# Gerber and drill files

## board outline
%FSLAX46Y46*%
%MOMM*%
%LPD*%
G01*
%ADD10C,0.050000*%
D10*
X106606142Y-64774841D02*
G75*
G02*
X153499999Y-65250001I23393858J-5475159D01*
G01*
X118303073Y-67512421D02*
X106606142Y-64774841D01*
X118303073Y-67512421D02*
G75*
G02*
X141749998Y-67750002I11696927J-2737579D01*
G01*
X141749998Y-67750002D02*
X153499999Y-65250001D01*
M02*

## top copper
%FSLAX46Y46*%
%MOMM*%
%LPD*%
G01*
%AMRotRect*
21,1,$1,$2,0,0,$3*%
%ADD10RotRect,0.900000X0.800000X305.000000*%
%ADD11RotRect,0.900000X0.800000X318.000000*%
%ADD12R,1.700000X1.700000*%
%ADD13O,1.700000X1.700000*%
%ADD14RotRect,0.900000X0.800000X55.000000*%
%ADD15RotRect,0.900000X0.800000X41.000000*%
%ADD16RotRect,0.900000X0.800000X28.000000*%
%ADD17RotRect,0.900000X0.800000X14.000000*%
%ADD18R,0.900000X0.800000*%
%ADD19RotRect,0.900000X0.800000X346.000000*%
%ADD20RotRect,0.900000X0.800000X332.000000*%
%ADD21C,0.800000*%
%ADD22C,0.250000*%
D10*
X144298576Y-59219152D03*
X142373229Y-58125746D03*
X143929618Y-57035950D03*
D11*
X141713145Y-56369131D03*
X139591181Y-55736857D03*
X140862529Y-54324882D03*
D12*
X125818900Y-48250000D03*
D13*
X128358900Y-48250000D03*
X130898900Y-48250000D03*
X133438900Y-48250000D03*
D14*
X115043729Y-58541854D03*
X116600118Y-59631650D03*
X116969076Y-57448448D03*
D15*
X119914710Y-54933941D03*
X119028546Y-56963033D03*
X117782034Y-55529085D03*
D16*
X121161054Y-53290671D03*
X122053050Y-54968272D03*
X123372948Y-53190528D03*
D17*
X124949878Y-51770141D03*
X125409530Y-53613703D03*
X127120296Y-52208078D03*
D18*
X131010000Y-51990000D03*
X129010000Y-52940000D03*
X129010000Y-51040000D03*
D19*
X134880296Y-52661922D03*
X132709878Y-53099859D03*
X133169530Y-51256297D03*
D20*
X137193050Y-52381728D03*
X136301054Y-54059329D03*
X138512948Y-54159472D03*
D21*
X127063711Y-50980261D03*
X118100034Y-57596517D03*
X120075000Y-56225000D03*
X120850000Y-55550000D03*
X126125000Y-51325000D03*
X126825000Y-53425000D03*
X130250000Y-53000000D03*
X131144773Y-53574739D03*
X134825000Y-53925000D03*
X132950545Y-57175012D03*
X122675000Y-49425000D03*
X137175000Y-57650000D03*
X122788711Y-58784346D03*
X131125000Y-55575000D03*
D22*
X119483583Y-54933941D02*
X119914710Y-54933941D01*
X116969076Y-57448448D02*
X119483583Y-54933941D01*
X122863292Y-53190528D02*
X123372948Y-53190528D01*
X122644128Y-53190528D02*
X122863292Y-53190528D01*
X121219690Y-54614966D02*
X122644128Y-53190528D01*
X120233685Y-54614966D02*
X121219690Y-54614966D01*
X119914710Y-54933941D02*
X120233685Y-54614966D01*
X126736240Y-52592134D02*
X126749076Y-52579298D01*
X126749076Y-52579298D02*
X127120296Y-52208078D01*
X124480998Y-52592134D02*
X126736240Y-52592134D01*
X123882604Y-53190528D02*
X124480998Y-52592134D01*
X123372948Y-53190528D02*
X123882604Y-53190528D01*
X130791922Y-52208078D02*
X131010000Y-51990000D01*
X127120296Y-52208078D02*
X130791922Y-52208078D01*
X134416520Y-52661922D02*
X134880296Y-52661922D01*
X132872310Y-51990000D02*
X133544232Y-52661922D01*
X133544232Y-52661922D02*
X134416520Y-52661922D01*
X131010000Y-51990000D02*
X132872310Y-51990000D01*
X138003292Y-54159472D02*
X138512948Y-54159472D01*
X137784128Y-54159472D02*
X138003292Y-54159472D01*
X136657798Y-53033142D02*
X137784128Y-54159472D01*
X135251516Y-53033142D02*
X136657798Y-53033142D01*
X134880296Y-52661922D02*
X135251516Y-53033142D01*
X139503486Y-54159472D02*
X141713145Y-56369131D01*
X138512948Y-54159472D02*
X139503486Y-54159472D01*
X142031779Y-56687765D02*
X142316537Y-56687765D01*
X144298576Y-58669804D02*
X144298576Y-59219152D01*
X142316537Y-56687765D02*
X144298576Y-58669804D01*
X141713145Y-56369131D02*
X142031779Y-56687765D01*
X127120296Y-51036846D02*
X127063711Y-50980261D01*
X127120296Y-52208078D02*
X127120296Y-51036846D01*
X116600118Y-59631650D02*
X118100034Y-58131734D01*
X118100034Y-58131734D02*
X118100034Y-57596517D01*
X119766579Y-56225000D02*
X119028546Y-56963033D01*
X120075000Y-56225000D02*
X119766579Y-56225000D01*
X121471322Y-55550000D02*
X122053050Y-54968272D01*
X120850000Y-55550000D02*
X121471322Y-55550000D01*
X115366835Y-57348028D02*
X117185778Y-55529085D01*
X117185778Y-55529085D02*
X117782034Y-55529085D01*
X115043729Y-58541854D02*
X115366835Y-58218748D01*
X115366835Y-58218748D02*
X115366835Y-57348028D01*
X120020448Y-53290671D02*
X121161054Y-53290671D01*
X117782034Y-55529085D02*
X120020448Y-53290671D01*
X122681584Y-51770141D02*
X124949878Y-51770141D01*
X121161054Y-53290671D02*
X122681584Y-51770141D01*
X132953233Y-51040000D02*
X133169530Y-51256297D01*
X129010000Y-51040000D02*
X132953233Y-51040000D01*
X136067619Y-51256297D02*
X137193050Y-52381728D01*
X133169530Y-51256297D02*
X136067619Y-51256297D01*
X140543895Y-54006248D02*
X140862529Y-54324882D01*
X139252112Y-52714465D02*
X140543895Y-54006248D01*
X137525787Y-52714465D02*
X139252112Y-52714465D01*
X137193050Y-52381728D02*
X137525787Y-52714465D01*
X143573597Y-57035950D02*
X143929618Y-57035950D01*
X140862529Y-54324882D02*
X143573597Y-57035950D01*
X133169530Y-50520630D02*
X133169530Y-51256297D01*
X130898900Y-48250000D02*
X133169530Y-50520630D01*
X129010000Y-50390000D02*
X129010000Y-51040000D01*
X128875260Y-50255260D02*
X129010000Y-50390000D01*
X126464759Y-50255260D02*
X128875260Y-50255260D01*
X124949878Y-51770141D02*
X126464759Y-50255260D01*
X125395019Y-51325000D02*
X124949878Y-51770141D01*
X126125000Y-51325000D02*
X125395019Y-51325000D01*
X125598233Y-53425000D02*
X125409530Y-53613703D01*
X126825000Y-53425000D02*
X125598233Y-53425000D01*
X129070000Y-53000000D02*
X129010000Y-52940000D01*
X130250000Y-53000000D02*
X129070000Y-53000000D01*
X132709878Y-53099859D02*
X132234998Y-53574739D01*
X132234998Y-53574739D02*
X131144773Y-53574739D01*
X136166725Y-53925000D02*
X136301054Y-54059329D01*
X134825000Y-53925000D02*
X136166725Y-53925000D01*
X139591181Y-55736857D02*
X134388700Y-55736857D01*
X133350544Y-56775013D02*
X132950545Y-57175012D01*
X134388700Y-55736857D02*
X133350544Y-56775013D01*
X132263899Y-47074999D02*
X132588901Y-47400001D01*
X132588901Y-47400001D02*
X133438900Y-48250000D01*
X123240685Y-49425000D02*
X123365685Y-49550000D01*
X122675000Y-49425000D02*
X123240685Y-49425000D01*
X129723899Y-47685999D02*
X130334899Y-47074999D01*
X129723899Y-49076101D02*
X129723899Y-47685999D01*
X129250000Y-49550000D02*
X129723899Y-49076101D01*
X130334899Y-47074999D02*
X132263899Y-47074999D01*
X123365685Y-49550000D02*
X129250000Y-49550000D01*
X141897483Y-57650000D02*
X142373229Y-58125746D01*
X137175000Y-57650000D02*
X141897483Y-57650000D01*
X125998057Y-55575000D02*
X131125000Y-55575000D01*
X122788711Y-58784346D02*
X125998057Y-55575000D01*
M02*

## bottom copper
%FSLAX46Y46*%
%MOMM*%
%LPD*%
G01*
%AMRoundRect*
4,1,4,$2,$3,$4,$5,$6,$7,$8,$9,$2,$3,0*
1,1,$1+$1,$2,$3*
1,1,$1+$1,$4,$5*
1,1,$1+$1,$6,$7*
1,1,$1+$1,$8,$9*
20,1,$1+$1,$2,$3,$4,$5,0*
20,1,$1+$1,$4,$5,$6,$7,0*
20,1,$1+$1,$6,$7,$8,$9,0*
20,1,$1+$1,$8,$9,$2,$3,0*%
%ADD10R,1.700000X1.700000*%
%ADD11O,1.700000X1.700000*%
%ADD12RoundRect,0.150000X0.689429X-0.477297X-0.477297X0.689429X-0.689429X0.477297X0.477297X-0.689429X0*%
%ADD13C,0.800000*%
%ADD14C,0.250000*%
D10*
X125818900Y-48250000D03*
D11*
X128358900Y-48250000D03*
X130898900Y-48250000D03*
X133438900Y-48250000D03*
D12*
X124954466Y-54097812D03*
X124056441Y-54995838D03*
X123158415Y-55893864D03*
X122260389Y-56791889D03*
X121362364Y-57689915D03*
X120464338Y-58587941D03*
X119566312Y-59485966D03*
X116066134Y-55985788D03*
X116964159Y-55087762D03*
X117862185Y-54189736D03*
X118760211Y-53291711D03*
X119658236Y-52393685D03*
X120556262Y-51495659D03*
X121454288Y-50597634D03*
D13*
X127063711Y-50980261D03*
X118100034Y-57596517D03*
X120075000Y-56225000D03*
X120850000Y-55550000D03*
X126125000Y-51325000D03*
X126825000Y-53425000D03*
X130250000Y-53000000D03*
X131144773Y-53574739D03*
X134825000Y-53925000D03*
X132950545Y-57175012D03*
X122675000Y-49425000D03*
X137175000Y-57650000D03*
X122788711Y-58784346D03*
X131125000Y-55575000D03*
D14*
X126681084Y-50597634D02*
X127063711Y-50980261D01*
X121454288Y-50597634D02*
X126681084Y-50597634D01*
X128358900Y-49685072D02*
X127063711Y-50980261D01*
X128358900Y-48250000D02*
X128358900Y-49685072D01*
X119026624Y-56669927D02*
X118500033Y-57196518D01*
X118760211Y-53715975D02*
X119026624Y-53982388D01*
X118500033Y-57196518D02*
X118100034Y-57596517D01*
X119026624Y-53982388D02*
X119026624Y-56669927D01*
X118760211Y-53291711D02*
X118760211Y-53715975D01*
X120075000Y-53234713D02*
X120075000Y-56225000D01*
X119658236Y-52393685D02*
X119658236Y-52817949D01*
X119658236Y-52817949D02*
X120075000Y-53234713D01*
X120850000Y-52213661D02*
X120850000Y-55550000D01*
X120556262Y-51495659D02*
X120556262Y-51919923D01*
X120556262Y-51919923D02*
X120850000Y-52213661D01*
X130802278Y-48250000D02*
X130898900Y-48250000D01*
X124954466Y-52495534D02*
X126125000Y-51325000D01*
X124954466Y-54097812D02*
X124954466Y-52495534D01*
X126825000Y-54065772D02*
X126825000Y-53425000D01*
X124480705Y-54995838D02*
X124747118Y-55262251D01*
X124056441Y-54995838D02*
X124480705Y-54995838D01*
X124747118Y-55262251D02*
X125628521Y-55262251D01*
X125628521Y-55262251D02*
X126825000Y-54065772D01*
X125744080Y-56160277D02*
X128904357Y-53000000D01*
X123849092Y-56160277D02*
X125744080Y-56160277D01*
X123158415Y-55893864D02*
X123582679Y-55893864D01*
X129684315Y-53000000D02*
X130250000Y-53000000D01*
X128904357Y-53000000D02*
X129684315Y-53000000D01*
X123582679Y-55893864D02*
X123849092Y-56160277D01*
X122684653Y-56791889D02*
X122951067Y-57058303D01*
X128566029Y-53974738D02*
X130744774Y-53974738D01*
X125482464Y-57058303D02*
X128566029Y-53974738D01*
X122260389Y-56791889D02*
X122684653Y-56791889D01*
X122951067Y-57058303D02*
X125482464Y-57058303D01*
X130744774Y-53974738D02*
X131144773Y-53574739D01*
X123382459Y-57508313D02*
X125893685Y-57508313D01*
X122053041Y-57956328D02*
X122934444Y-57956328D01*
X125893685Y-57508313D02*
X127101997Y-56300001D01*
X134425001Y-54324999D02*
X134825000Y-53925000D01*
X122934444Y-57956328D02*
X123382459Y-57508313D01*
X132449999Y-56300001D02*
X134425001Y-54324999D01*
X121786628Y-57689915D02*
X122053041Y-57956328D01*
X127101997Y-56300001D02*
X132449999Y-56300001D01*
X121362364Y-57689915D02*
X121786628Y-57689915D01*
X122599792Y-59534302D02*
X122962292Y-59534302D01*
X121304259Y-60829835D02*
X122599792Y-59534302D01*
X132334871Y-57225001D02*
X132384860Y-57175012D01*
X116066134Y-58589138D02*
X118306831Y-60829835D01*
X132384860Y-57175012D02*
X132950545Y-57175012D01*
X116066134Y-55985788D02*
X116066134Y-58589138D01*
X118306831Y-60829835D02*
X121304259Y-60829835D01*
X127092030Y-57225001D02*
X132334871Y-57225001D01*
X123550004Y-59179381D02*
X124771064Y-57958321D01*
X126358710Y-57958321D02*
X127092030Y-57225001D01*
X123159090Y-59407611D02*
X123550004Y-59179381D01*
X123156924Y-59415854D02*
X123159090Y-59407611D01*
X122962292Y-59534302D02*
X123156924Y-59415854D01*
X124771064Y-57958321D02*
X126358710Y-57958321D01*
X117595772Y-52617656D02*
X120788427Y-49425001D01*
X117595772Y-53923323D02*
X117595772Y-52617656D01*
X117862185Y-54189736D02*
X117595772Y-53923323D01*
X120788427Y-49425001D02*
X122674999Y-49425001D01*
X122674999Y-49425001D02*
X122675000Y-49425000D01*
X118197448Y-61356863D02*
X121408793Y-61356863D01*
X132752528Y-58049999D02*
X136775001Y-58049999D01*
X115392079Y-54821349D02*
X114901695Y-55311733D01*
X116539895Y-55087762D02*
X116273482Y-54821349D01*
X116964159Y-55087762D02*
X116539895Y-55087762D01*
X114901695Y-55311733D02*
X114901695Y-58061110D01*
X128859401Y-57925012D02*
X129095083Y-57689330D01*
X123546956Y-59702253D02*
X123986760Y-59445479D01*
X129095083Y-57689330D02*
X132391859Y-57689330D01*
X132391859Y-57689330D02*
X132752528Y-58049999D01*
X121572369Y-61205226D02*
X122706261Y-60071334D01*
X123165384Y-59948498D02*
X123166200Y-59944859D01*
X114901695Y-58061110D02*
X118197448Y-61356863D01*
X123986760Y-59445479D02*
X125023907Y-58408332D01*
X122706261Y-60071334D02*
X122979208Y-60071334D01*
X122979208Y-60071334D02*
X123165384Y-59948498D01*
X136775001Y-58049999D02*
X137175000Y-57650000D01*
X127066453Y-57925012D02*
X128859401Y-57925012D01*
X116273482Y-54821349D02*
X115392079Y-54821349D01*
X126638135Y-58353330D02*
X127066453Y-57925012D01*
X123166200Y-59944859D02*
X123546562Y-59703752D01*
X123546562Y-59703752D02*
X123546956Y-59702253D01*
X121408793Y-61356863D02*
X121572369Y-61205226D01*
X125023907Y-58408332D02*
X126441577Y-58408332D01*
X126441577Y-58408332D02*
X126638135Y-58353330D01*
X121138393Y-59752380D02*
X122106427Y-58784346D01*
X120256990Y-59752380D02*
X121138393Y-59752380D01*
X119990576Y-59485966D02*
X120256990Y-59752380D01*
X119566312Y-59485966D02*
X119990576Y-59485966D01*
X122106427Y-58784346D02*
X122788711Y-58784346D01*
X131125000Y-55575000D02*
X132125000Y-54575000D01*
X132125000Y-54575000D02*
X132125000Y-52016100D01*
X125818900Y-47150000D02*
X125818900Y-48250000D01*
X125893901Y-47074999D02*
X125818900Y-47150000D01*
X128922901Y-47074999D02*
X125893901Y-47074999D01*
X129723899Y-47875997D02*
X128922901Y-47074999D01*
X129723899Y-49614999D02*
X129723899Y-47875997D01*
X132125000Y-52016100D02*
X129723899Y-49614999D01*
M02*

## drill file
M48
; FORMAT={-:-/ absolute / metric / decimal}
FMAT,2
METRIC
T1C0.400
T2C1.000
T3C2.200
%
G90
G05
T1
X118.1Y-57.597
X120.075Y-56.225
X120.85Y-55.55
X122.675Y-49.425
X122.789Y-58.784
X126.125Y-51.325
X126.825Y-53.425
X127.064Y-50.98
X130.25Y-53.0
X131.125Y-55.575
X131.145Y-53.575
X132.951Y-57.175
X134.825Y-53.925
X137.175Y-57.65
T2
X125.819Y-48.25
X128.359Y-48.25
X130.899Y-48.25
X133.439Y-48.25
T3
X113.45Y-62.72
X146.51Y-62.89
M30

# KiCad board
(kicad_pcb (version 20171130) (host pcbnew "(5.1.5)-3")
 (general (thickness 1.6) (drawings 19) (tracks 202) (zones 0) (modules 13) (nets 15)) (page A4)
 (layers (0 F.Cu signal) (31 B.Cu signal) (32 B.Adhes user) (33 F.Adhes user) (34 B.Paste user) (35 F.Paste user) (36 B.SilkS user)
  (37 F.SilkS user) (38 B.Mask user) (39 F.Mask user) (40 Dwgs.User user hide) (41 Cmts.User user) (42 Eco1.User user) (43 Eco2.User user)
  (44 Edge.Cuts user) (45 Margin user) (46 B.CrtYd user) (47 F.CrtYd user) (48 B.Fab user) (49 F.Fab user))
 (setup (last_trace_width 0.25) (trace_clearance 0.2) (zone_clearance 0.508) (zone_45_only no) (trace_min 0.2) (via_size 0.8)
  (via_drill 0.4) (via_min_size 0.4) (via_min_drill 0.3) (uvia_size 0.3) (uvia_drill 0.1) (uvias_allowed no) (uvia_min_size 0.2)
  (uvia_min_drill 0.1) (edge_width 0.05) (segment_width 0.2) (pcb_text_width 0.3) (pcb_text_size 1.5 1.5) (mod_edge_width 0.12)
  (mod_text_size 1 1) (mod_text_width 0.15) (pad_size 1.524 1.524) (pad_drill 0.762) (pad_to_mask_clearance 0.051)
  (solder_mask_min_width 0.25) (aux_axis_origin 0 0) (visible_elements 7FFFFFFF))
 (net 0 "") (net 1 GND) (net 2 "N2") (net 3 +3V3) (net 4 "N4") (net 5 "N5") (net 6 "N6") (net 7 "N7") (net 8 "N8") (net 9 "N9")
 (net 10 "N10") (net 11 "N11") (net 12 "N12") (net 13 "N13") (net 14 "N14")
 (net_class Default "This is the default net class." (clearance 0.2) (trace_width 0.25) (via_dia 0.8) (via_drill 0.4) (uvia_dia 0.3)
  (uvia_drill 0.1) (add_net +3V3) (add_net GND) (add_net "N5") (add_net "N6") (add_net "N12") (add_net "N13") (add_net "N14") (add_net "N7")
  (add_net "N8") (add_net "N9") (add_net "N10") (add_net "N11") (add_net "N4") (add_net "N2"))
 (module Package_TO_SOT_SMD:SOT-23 (layer F.Cu) (at 143.725 58.4 305)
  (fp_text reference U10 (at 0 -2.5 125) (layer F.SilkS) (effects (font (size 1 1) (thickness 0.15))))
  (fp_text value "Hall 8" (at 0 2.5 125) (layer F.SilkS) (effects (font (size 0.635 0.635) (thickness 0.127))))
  (pad 3 smd rect (at 1 0 305) (size 0.9 0.8) (layers F.Cu F.Paste F.Mask) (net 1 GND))
  (pad 2 smd rect (at -1 0.95 305) (size 0.9 0.8) (layers F.Cu F.Paste F.Mask) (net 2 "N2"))
  (pad 1 smd rect (at -1 -0.95 305) (size 0.9 0.8) (layers F.Cu F.Paste F.Mask) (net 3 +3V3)))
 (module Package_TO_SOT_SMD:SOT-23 (layer F.Cu) (at 140.97 55.7 318)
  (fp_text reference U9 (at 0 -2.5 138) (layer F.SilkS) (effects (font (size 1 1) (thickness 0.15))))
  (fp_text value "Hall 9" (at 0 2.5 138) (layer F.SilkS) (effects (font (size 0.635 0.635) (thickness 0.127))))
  (pad 3 smd rect (at 1 0 318) (size 0.9 0.8) (layers F.Cu F.Paste F.Mask) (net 1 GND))
  (pad 2 smd rect (at -1 0.95 318) (size 0.9 0.8) (layers F.Cu F.Paste F.Mask) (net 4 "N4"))
  (pad 1 smd rect (at -1 -0.95 318) (size 0.9 0.8) (layers F.Cu F.Paste F.Mask) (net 3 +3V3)))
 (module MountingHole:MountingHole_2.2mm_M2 (layer F.Cu) (at 146.51 62.89)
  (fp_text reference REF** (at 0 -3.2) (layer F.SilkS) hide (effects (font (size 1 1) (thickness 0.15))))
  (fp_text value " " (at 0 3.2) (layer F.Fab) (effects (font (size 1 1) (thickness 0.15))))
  (pad 1 np_thru_hole circle (at 0 0) (size 2.2 2.2) (drill 2.2) (layers *.Cu *.Mask)))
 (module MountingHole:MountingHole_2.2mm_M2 (layer F.Cu) (at 113.45 62.72)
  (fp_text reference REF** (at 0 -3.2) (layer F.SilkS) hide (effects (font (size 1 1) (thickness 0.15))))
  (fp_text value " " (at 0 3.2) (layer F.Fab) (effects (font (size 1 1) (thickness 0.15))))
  (pad 1 np_thru_hole circle (at 0 0) (size 2.2 2.2) (drill 2.2) (layers *.Cu *.Mask)))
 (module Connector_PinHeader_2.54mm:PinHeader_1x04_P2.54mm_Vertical (layer F.Cu) (at 125.8189 48.25 90)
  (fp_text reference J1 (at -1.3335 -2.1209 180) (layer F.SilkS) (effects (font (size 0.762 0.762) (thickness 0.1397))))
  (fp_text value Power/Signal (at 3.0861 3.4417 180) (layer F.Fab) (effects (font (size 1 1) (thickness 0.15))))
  (pad 1 thru_hole rect (at 0 0 90) (size 1.7 1.7) (drill 1) (layers *.Cu *.Mask) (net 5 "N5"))
  (pad 2 thru_hole oval (at 0 2.54 90) (size 1.7 1.7) (drill 1) (layers *.Cu *.Mask) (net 1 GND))
  (pad 3 thru_hole oval (at 0 5.08 90) (size 1.7 1.7) (drill 1) (layers *.Cu *.Mask) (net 3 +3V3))
  (pad 4 thru_hole oval (at 0 7.62 90) (size 1.7 1.7) (drill 1) (layers *.Cu *.Mask) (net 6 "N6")))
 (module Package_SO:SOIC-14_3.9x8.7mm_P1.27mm (layer B.Cu) (at 120.5103 55.0418 135)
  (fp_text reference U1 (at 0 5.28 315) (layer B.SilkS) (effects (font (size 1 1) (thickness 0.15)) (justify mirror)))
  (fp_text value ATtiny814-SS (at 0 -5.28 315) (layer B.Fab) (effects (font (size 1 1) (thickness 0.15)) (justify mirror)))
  (pad 1 smd roundrect (at -2.475 3.81 135) (size 1.95 0.6) (layers B.Cu B.Paste B.Mask) (roundrect_rratio 0.25) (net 3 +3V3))
  (pad 2 smd roundrect (at -2.475 2.54 135) (size 1.95 0.6) (layers B.Cu B.Paste B.Mask) (roundrect_rratio 0.25) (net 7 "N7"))
  (pad 3 smd roundrect (at -2.475 1.27 135) (size 1.95 0.6) (layers B.Cu B.Paste B.Mask) (roundrect_rratio 0.25) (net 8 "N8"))
  (pad 4 smd roundrect (at -2.475 0 135) (size 1.95 0.6) (layers B.Cu B.Paste B.Mask) (roundrect_rratio 0.25) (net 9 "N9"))
  (pad 5 smd roundrect (at -2.475 -1.27 135) (size 1.95 0.6) (layers B.Cu B.Paste B.Mask) (roundrect_rratio 0.25) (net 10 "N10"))
  (pad 6 smd roundrect (at -2.475 -2.54 135) (size 1.95 0.6) (layers B.Cu B.Paste B.Mask) (roundrect_rratio 0.25) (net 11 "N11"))
  (pad 7 smd roundrect (at -2.475 -3.81 135) (size 1.95 0.6) (layers B.Cu B.Paste B.Mask) (roundrect_rratio 0.25) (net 5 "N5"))
  (pad 8 smd roundrect (at 2.475 -3.81 135) (size 1.95 0.6) (layers B.Cu B.Paste B.Mask) (roundrect_rratio 0.25) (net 4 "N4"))
  (pad 9 smd roundrect (at 2.475 -2.54 135) (size 1.95 0.6) (layers B.Cu B.Paste B.Mask) (roundrect_rratio 0.25) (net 2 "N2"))
  (pad 10 smd roundrect (at 2.475 -1.27 135) (size 1.95 0.6) (layers B.Cu B.Paste B.Mask) (roundrect_rratio 0.25) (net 6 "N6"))
  (pad 11 smd roundrect (at 2.475 0 135) (size 1.95 0.6) (layers B.Cu B.Paste B.Mask) (roundrect_rratio 0.25) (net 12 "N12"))
  (pad 12 smd roundrect (at 2.475 1.27 135) (size 1.95 0.6) (layers B.Cu B.Paste B.Mask) (roundrect_rratio 0.25) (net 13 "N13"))
  (pad 13 smd roundrect (at 2.475 2.54 135) (size 1.95 0.6) (layers B.Cu B.Paste B.Mask) (roundrect_rratio 0.25) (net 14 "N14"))
  (pad 14 smd roundrect (at 2.475 3.81 135) (size 1.95 0.6) (layers B.Cu B.Paste B.Mask) (roundrect_rratio 0.25) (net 1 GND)))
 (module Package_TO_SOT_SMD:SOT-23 (layer F.Cu) (at 116.3955 58.2676 55)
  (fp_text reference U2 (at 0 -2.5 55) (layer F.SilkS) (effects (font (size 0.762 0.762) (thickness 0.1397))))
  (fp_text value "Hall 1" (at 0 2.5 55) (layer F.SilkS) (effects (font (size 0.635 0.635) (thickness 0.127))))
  (pad 1 smd rect (at -1 -0.95 55) (size 0.9 0.8) (layers F.Cu F.Paste F.Mask) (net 3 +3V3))
  (pad 2 smd rect (at -1 0.95 55) (size 0.9 0.8) (layers F.Cu F.Paste F.Mask) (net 12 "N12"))
  (pad 3 smd rect (at 1 0 55) (size 0.9 0.8) (layers F.Cu F.Paste F.Mask) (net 1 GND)))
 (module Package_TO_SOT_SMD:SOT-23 (layer F.Cu) (at 119.16 55.59 41)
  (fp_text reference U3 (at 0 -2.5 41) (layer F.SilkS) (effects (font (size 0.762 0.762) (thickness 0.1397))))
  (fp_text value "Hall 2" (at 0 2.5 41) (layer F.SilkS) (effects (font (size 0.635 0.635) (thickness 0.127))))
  (pad 3 smd rect (at 1 0 41) (size 0.9 0.8) (layers F.Cu F.Paste F.Mask) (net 1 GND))
  (pad 2 smd rect (at -1 0.95 41) (size 0.9 0.8) (layers F.Cu F.Paste F.Mask) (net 13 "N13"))
  (pad 1 smd rect (at -1 -0.95 41) (size 0.9 0.8) (layers F.Cu F.Paste F.Mask) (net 3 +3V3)))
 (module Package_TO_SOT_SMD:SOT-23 (layer F.Cu) (at 122.49 53.66 28)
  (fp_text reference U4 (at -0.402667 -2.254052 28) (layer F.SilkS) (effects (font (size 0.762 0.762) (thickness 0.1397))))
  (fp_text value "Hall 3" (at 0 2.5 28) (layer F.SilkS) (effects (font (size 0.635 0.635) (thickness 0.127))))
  (pad 1 smd rect (at -1 -0.95 28) (size 0.9 0.8) (layers F.Cu F.Paste F.Mask) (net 3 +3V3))
  (pad 2 smd rect (at -1 0.95 28) (size 0.9 0.8) (layers F.Cu F.Paste F.Mask) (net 14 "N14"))
  (pad 3 smd rect (at 1 0 28) (size 0.9 0.8) (layers F.Cu F.Paste F.Mask) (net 1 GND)))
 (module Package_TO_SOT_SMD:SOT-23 (layer F.Cu) (at 126.15 52.45 14)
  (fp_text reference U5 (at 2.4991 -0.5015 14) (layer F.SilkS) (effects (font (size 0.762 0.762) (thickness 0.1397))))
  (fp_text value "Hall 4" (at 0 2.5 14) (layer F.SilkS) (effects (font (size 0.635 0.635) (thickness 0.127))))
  (pad 1 smd rect (at -1 -0.95 14) (size 0.9 0.8) (layers F.Cu F.Paste F.Mask) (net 3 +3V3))
  (pad 2 smd rect (at -1 0.95 14) (size 0.9 0.8) (layers F.Cu F.Paste F.Mask) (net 7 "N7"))
  (pad 3 smd rect (at 1 0 14) (size 0.9 0.8) (layers F.Cu F.Paste F.Mask) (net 1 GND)))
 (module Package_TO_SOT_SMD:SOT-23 (layer F.Cu) (at 130.01 51.99)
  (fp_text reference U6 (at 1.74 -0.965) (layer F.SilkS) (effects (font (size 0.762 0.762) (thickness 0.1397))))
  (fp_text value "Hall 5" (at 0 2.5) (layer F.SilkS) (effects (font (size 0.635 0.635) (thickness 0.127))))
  (pad 3 smd rect (at 1 0) (size 0.9 0.8) (layers F.Cu F.Paste F.Mask) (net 1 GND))
  (pad 2 smd rect (at -1 0.95) (size 0.9 0.8) (layers F.Cu F.Paste F.Mask) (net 8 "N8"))
  (pad 1 smd rect (at -1 -0.95) (size 0.9 0.8) (layers F.Cu F.Paste F.Mask) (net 3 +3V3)))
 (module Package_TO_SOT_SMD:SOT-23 (layer F.Cu) (at 133.91 52.42 346)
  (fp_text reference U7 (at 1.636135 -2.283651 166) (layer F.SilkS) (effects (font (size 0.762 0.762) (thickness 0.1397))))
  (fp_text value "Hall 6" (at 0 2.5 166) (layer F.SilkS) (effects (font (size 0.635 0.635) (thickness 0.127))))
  (pad 3 smd rect (at 1 0 346) (size 0.9 0.8) (layers F.Cu F.Paste F.Mask) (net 1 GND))
  (pad 2 smd rect (at -1 0.95 346) (size 0.9 0.8) (layers F.Cu F.Paste F.Mask) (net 9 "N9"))
  (pad 1 smd rect (at -1 -0.95 346) (size 0.9 0.8) (layers F.Cu F.Paste F.Mask) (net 3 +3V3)))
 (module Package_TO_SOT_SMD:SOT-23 (layer F.Cu) (at 137.63 53.69 332)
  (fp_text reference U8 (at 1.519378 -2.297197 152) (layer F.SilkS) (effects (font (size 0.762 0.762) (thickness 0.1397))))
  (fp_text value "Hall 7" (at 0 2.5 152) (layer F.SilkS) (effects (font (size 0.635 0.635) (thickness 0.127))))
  (pad 1 smd rect (at -1 -0.95 332) (size 0.9 0.8) (layers F.Cu F.Paste F.Mask) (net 3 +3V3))
  (pad 2 smd rect (at -1 0.95 332) (size 0.9 0.8) (layers F.Cu F.Paste F.Mask) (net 10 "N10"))
  (pad 3 smd rect (at 1 0 332) (size 0.9 0.8) (layers F.Cu F.Paste F.Mask) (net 1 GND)))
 (gr_arc (start 130 70.25) (end 153.499999 65.250001) (angle -154.8159682) (layer Edge.Cuts) (width 0.05))
 (gr_line (start 118.303073 67.512421) (end 106.606142 64.774841) (layer Edge.Cuts) (width 0.05))
 (gr_arc (start 130 70.25) (end 141.749998 67.750002) (angle -154.8159719) (layer Edge.Cuts) (width 0.05))
 (gr_line (start 141.749998 67.750002) (end 153.499999 65.250001) (layer Edge.Cuts) (width 0.05))
 (segment (start 119.483583 54.933941) (end 119.91471 54.933941) (width 0.25) (layer F.Cu) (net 1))
 (segment (start 116.969076 57.448448) (end 119.483583 54.933941) (width 0.25) (layer F.Cu) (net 1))
 (segment (start 122.863292 53.190528) (end 123.372948 53.190528) (width 0.25) (layer F.Cu) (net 1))
 (segment (start 122.644128 53.190528) (end 122.863292 53.190528) (width 0.25) (layer F.Cu) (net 1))
 (segment (start 121.21969 54.614966) (end 122.644128 53.190528) (width 0.25) (layer F.Cu) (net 1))
 (segment (start 120.233685 54.614966) (end 121.21969 54.614966) (width 0.25) (layer F.Cu) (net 1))
 (segment (start 119.91471 54.933941) (end 120.233685 54.614966) (width 0.25) (layer F.Cu) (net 1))
 (segment (start 126.73624 52.592134) (end 126.749076 52.579298) (width 0.25) (layer F.Cu) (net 1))
 (segment (start 126.749076 52.579298) (end 127.120296 52.208078) (width 0.25) (layer F.Cu) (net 1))
 (segment (start 124.480998 52.592134) (end 126.73624 52.592134) (width 0.25) (layer F.Cu) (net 1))
 (segment (start 123.882604 53.190528) (end 124.480998 52.592134) (width 0.25) (layer F.Cu) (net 1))
 (segment (start 123.372948 53.190528) (end 123.882604 53.190528) (width 0.25) (layer F.Cu) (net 1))
 (segment (start 130.791922 52.208078) (end 131.01 51.99) (width 0.25) (layer F.Cu) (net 1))
 (segment (start 127.120296 52.208078) (end 130.791922 52.208078) (width 0.25) (layer F.Cu) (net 1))
 (segment (start 134.41652 52.661922) (end 134.880296 52.661922) (width 0.25) (layer F.Cu) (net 1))
 (segment (start 132.87231 51.99) (end 133.544232 52.661922) (width 0.25) (layer F.Cu) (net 1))
 (segment (start 133.544232 52.661922) (end 134.41652 52.661922) (width 0.25) (layer F.Cu) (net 1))
 (segment (start 131.01 51.99) (end 132.87231 51.99) (width 0.25) (layer F.Cu) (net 1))
 (segment (start 138.003292 54.159472) (end 138.512948 54.159472) (width 0.25) (layer F.Cu) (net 1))
 (segment (start 137.784128 54.159472) (end 138.003292 54.159472) (width 0.25) (layer F.Cu) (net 1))
 (segment (start 136.657798 53.033142) (end 137.784128 54.159472) (width 0.25) (layer F.Cu) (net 1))
 (segment (start 135.251516 53.033142) (end 136.657798 53.033142) (width 0.25) (layer F.Cu) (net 1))
 (segment (start 134.880296 52.661922) (end 135.251516 53.033142) (width 0.25) (layer F.Cu) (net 1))
 (segment (start 139.503486 54.159472) (end 141.713145 56.369131) (width 0.25) (layer F.Cu) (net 1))
 (segment (start 138.512948 54.159472) (end 139.503486 54.159472) (width 0.25) (layer F.Cu) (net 1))
 (segment (start 142.031779 56.687765) (end 142.316537 56.687765) (width 0.25) (layer F.Cu) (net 1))
 (segment (start 144.298576 58.669804) (end 144.298576 59.219152) (width 0.25) (layer F.Cu) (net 1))
 (segment (start 142.316537 56.687765) (end 144.298576 58.669804) (width 0.25) (layer F.Cu) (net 1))
 (segment (start 141.713145 56.369131) (end 142.031779 56.687765) (width 0.25) (layer F.Cu) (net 1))
 (via (at 127.063711 50.980261) (size 0.8) (drill 0.4) (layers F.Cu B.Cu) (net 1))
 (segment (start 127.120296 51.036846) (end 127.063711 50.980261) (width 0.25) (layer F.Cu) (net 1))
 (segment (start 127.120296 52.208078) (end 127.120296 51.036846) (width 0.25) (layer F.Cu) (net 1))
 (segment (start 126.681084 50.597634) (end 127.063711 50.980261) (width 0.25) (layer B.Cu) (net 1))
 (segment (start 121.454288 50.597634) (end 126.681084 50.597634) (width 0.25) (layer B.Cu) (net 1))
 (segment (start 128.3589 49.685072) (end 127.063711 50.980261) (width 0.25) (layer B.Cu) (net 1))
 (segment (start 128.3589 48.25) (end 128.3589 49.685072) (width 0.25) (layer B.Cu) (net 1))
 (segment (start 116.600118 59.63165) (end 118.100034 58.131734) (width 0.25) (layer F.Cu) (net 12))
 (via (at 118.100034 57.596517) (size 0.8) (drill 0.4) (layers F.Cu B.Cu) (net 12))
 (segment (start 118.100034 58.131734) (end 118.100034 57.596517) (width 0.25) (layer F.Cu) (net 12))
 (segment (start 119.026624 56.669927) (end 118.500033 57.196518) (width 0.25) (layer B.Cu) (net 12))
 (segment (start 118.760211 53.715975) (end 119.026624 53.982388) (width 0.25) (layer B.Cu) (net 12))
 (segment (start 118.500033 57.196518) (end 118.100034 57.596517) (width 0.25) (layer B.Cu) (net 12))
 (segment (start 119.026624 53.982388) (end 119.026624 56.669927) (width 0.25) (layer B.Cu) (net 12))
 (segment (start 118.760211 53.291711) (end 118.760211 53.715975) (width 0.25) (layer B.Cu) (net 12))
 (via (at 120.075 56.225) (size 0.8) (drill 0.4) (layers F.Cu B.Cu) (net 13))
 (segment (start 120.075 53.234713) (end 120.075 56.225) (width 0.25) (layer B.Cu) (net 13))
 (segment (start 119.658236 52.393685) (end 119.658236 52.817949) (width 0.25) (layer B.Cu) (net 13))
 (segment (start 119.658236 52.817949) (end 120.075 53.234713) (width 0.25) (layer B.Cu) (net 13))
 (segment (start 119.766579 56.225) (end 119.028546 56.963033) (width 0.25) (layer F.Cu) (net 13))
 (segment (start 120.075 56.225) (end 119.766579 56.225) (width 0.25) (layer F.Cu) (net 13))
 (segment (start 120.85 52.213661) (end 120.85 55.55) (width 0.25) (layer B.Cu) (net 14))
 (via (at 120.85 55.55) (size 0.8) (drill 0.4) (layers F.Cu B.Cu) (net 14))
 (segment (start 120.556262 51.495659) (end 120.556262 51.919923) (width 0.25) (layer B.Cu) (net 14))
 (segment (start 120.556262 51.919923) (end 120.85 52.213661) (width 0.25) (layer B.Cu) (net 14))
 (segment (start 121.471322 55.55) (end 122.05305 54.968272) (width 0.25) (layer F.Cu) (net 14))
 (segment (start 120.85 55.55) (end 121.471322 55.55) (width 0.25) (layer F.Cu) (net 14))
 (segment (start 115.366835 57.348028) (end 117.185778 55.529085) (width 0.25) (layer F.Cu) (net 3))
 (segment (start 117.185778 55.529085) (end 117.782034 55.529085) (width 0.25) (layer F.Cu) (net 3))
 (segment (start 115.043729 58.541854) (end 115.366835 58.218748) (width 0.25) (layer F.Cu) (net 3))
 (segment (start 115.366835 58.218748) (end 115.366835 57.348028) (width 0.25) (layer F.Cu) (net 3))
 (segment (start 120.020448 53.290671) (end 121.161054 53.290671) (width 0.25) (layer F.Cu) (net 3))
 (segment (start 117.782034 55.529085) (end 120.020448 53.290671) (width 0.25) (layer F.Cu) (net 3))
 (segment (start 122.681584 51.770141) (end 124.949878 51.770141) (width 0.25) (layer F.Cu) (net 3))
 (segment (start 121.161054 53.290671) (end 122.681584 51.770141) (width 0.25) (layer F.Cu) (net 3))
 (segment (start 132.953233 51.04) (end 133.16953 51.256297) (width 0.25) (layer F.Cu) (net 3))
 (segment (start 129.01 51.04) (end 132.953233 51.04) (width 0.25) (layer F.Cu) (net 3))
 (segment (start 136.067619 51.256297) (end 137.19305 52.381728) (width 0.25) (layer F.Cu) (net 3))
 (segment (start 133.16953 51.256297) (end 136.067619 51.256297) (width 0.25) (layer F.Cu) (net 3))
 (segment (start 140.543895 54.006248) (end 140.862529 54.324882) (width 0.25) (layer F.Cu) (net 3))
 (segment (start 139.252112 52.714465) (end 140.543895 54.006248) (width 0.25) (layer F.Cu) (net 3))
 (segment (start 137.525787 52.714465) (end 139.252112 52.714465) (width 0.25) (layer F.Cu) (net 3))
 (segment (start 137.19305 52.381728) (end 137.525787 52.714465) (width 0.25) (layer F.Cu) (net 3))
 (segment (start 143.573597 57.03595) (end 143.929618 57.03595) (width 0.25) (layer F.Cu) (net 3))
 (segment (start 140.862529 54.324882) (end 143.573597 57.03595) (width 0.25) (layer F.Cu) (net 3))
 (segment (start 130.802278 48.25) (end 130.8989 48.25) (width 0.25) (layer B.Cu) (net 3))
 (segment (start 133.16953 50.52063) (end 133.16953 51.256297) (width 0.25) (layer F.Cu) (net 3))
 (segment (start 130.8989 48.25) (end 133.16953 50.52063) (width 0.25) (layer F.Cu) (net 3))
 (via (at 126.125 51.325) (size 0.8) (drill 0.4) (layers F.Cu B.Cu) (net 3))
 (segment (start 124.954466 52.495534) (end 126.125 51.325) (width 0.25) (layer B.Cu) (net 3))
 (segment (start 124.954466 54.097812) (end 124.954466 52.495534) (width 0.25) (layer B.Cu) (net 3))
 (segment (start 129.01 50.39) (end 129.01 51.04) (width 0.25) (layer F.Cu) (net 3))
 (segment (start 128.87526 50.25526) (end 129.01 50.39) (width 0.25) (layer F.Cu) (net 3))
 (segment (start 126.464759 50.25526) (end 128.87526 50.25526) (width 0.25) (layer F.Cu) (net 3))
 (segment (start 124.949878 51.770141) (end 126.464759 50.25526) (width 0.25) (layer F.Cu) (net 3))
 (segment (start 125.395019 51.325) (end 124.949878 51.770141) (width 0.25) (layer F.Cu) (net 3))
 (segment (start 126.125 51.325) (end 125.395019 51.325) (width 0.25) (layer F.Cu) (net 3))
 (segment (start 126.825 54.065772) (end 126.825 53.425) (width 0.25) (layer B.Cu) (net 7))
 (via (at 126.825 53.425) (size 0.8) (drill 0.4) (layers F.Cu B.Cu) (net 7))
 (segment (start 124.480705 54.995838) (end 124.747118 55.262251) (width 0.25) (layer B.Cu) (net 7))
 (segment (start 124.056441 54.995838) (end 124.480705 54.995838) (width 0.25) (layer B.Cu) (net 7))
 (segment (start 124.747118 55.262251) (end 125.628521 55.262251) (width 0.25) (layer B.Cu) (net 7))
 (segment (start 125.628521 55.262251) (end 126.825 54.065772) (width 0.25) (layer B.Cu) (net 7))
 (segment (start 125.598233 53.425) (end 125.40953 53.613703) (width 0.25) (layer F.Cu) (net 7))
 (segment (start 126.825 53.425) (end 125.598233 53.425) (width 0.25) (layer F.Cu) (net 7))
 (via (at 130.25 53) (size 0.8) (drill 0.4) (layers F.Cu B.Cu) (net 8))
 (segment (start 129.07 53) (end 129.01 52.94) (width 0.25) (layer F.Cu) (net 8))
 (segment (start 130.25 53) (end 129.07 53) (width 0.25) (layer F.Cu) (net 8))
 (segment (start 125.74408 56.160277) (end 128.904357 53) (width 0.25) (layer B.Cu) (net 8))
 (segment (start 123.849092 56.160277) (end 125.74408 56.160277) (width 0.25) (layer B.Cu) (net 8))
 (segment (start 123.158415 55.893864) (end 123.582679 55.893864) (width 0.25) (layer B.Cu) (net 8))
 (segment (start 129.684315 53) (end 130.25 53) (width 0.25) (layer B.Cu) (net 8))
 (segment (start 128.904357 53) (end 129.684315 53) (width 0.25) (layer B.Cu) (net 8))
 (segment (start 123.582679 55.893864) (end 123.849092 56.160277) (width 0.25) (layer B.Cu) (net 8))
 (segment (start 122.684653 56.791889) (end 122.951067 57.058303) (width 0.25) (layer B.Cu) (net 9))
 (segment (start 128.566029 53.974738) (end 130.744774 53.974738) (width 0.25) (layer B.Cu) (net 9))
 (segment (start 132.709878 53.099859) (end 132.234998 53.574739) (width 0.25) (layer F.Cu) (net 9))
 (segment (start 125.482464 57.058303) (end 128.566029 53.974738) (width 0.25) (layer B.Cu) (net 9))
 (via (at 131.144773 53.574739) (size 0.8) (drill 0.4) (layers F.Cu B.Cu) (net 9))
 (segment (start 122.260389 56.791889) (end 122.684653 56.791889) (width 0.25) (layer B.Cu) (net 9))
 (segment (start 132.234998 53.574739) (end 131.144773 53.574739) (width 0.25) (layer F.Cu) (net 9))
 (segment (start 122.951067 57.058303) (end 125.482464 57.058303) (width 0.25) (layer B.Cu) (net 9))
 (segment (start 130.744774 53.974738) (end 131.144773 53.574739) (width 0.25) (layer B.Cu) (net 9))
 (via (at 134.825 53.925) (size 0.8) (drill 0.4) (layers F.Cu B.Cu) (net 10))
 (segment (start 136.166725 53.925) (end 136.301054 54.059329) (width 0.25) (layer F.Cu) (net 10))
 (segment (start 134.825 53.925) (end 136.166725 53.925) (width 0.25) (layer F.Cu) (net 10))
 (segment (start 123.382459 57.508313) (end 125.893685 57.508313) (width 0.25) (layer B.Cu) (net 10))
 (segment (start 122.053041 57.956328) (end 122.934444 57.956328) (width 0.25) (layer B.Cu) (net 10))
 (segment (start 125.893685 57.508313) (end 127.101997 56.300001) (width 0.25) (layer B.Cu) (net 10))
 (segment (start 134.425001 54.324999) (end 134.825 53.925) (width 0.25) (layer B.Cu) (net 10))
 (segment (start 122.934444 57.956328) (end 123.382459 57.508313) (width 0.25) (layer B.Cu) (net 10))
 (segment (start 132.449999 56.300001) (end 134.425001 54.324999) (width 0.25) (layer B.Cu) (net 10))
 (segment (start 121.786628 57.689915) (end 122.053041 57.956328) (width 0.25) (layer B.Cu) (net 10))
 (segment (start 127.101997 56.300001) (end 132.449999 56.300001) (width 0.25) (layer B.Cu) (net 10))
 (segment (start 121.362364 57.689915) (end 121.786628 57.689915) (width 0.25) (layer B.Cu) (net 10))
 (segment (start 139.591181 55.736857) (end 134.3887 55.736857) (width 0.25) (layer F.Cu) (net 4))
 (segment (start 133.350544 56.775013) (end 132.950545 57.175012) (width 0.25) (layer F.Cu) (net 4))
 (segment (start 134.3887 55.736857) (end 133.350544 56.775013) (width 0.25) (layer F.Cu) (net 4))
 (via (at 132.950545 57.175012) (size 0.8) (drill 0.4) (layers F.Cu B.Cu) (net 4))
 (segment (start 122.599792 59.534302) (end 122.962292 59.534302) (width 0.25) (layer B.Cu) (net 4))
 (segment (start 121.304259 60.829835) (end 122.599792 59.534302) (width 0.25) (layer B.Cu) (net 4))
 (segment (start 132.334871 57.225001) (end 132.38486 57.175012) (width 0.25) (layer B.Cu) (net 4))
 (segment (start 116.066134 58.589138) (end 118.306831 60.829835) (width 0.25) (layer B.Cu) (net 4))
 (segment (start 132.38486 57.175012) (end 132.950545 57.175012) (width 0.25) (layer B.Cu) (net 4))
 (segment (start 116.066134 55.985788) (end 116.066134 58.589138) (width 0.25) (layer B.Cu) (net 4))
 (segment (start 118.306831 60.829835) (end 121.304259 60.829835) (width 0.25) (layer B.Cu) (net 4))
 (segment (start 127.09203 57.225001) (end 132.334871 57.225001) (width 0.25) (layer B.Cu) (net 4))
 (segment (start 123.550004 59.179381) (end 124.771064 57.958321) (width 0.25) (layer B.Cu) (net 4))
 (segment (start 126.35871 57.958321) (end 127.09203 57.225001) (width 0.25) (layer B.Cu) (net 4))
 (segment (start 123.15909 59.407611) (end 123.550004 59.179381) (width 0.25) (layer B.Cu) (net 4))
 (segment (start 123.156924 59.415854) (end 123.15909 59.407611) (width 0.25) (layer B.Cu) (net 4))
 (segment (start 122.962292 59.534302) (end 123.156924 59.415854) (width 0.25) (layer B.Cu) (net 4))
 (segment (start 124.771064 57.958321) (end 126.35871 57.958321) (width 0.25) (layer B.Cu) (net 4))
 (segment (start 117.595772 52.617656) (end 120.788427 49.425001) (width 0.25) (layer B.Cu) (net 6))
 (segment (start 117.595772 53.923323) (end 117.595772 52.617656) (width 0.25) (layer B.Cu) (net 6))
 (segment (start 117.862185 54.189736) (end 117.595772 53.923323) (width 0.25) (layer B.Cu) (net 6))
 (via (at 122.675 49.425) (size 0.8) (drill 0.4) (layers F.Cu B.Cu) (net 6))
 (segment (start 120.788427 49.425001) (end 122.674999 49.425001) (width 0.25) (layer B.Cu) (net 6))
 (segment (start 122.674999 49.425001) (end 122.675 49.425) (width 0.25) (layer B.Cu) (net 6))
 (segment (start 132.263899 47.074999) (end 132.588901 47.400001) (width 0.25) (layer F.Cu) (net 6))
 (segment (start 132.588901 47.400001) (end 133.4389 48.25) (width 0.25) (layer F.Cu) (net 6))
 (segment (start 123.240685 49.425) (end 123.365685 49.55) (width 0.25) (layer F.Cu) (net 6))
 (segment (start 122.675 49.425) (end 123.240685 49.425) (width 0.25) (layer F.Cu) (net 6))
 (segment (start 129.723899 47.685999) (end 130.334899 47.074999) (width 0.25) (layer F.Cu) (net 6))
 (segment (start 129.723899 49.076101) (end 129.723899 47.685999) (width 0.25) (layer F.Cu) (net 6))
 (segment (start 129.25 49.55) (end 129.723899 49.076101) (width 0.25) (layer F.Cu) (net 6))
 (segment (start 130.334899 47.074999) (end 132.263899 47.074999) (width 0.25) (layer F.Cu) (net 6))
 (segment (start 123.365685 49.55) (end 129.25 49.55) (width 0.25) (layer F.Cu) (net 6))
 (via (at 137.175 57.65) (size 0.8) (drill 0.4) (layers F.Cu B.Cu) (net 2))
 (segment (start 141.897483 57.65) (end 142.373229 58.125746) (width 0.25) (layer F.Cu) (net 2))
 (segment (start 137.175 57.65) (end 141.897483 57.65) (width 0.25) (layer F.Cu) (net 2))
 (segment (start 118.197448 61.356863) (end 121.408793 61.356863) (width 0.25) (layer B.Cu) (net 2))
 (segment (start 132.752528 58.049999) (end 136.775001 58.049999) (width 0.25) (layer B.Cu) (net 2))
 (segment (start 115.392079 54.821349) (end 114.901695 55.311733) (width 0.25) (layer B.Cu) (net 2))
 (segment (start 116.539895 55.087762) (end 116.273482 54.821349) (width 0.25) (layer B.Cu) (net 2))
 (segment (start 116.964159 55.087762) (end 116.539895 55.087762) (width 0.25) (layer B.Cu) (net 2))
 (segment (start 114.901695 55.311733) (end 114.901695 58.06111) (width 0.25) (layer B.Cu) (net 2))
 (segment (start 128.859401 57.925012) (end 129.095083 57.68933) (width 0.25) (layer B.Cu) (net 2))
 (segment (start 123.546956 59.702253) (end 123.98676 59.445479) (width 0.25) (layer B.Cu) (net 2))
 (segment (start 129.095083 57.68933) (end 132.391859 57.68933) (width 0.25) (layer B.Cu) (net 2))
 (segment (start 132.391859 57.68933) (end 132.752528 58.049999) (width 0.25) (layer B.Cu) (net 2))
 (segment (start 121.572369 61.205226) (end 122.706261 60.071334) (width 0.25) (layer B.Cu) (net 2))
 (segment (start 123.165384 59.948498) (end 123.1662 59.944859) (width 0.25) (layer B.Cu) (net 2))
 (segment (start 114.901695 58.06111) (end 118.197448 61.356863) (width 0.25) (layer B.Cu) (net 2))
 (segment (start 123.98676 59.445479) (end 125.023907 58.408332) (width 0.25) (layer B.Cu) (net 2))
 (segment (start 122.706261 60.071334) (end 122.979208 60.071334) (width 0.25) (layer B.Cu) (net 2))
 (segment (start 122.979208 60.071334) (end 123.165384 59.948498) (width 0.25) (layer B.Cu) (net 2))
 (segment (start 136.775001 58.049999) (end 137.175 57.65) (width 0.25) (layer B.Cu) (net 2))
 (segment (start 127.066453 57.925012) (end 128.859401 57.925012) (width 0.25) (layer B.Cu) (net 2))
 (segment (start 116.273482 54.821349) (end 115.392079 54.821349) (width 0.25) (layer B.Cu) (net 2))
 (segment (start 126.638135 58.35333) (end 127.066453 57.925012) (width 0.25) (layer B.Cu) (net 2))
 (segment (start 123.1662 59.944859) (end 123.546562 59.703752) (width 0.25) (layer B.Cu) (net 2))
 (segment (start 123.546562 59.703752) (end 123.546956 59.702253) (width 0.25) (layer B.Cu) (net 2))
 (segment (start 121.408793 61.356863) (end 121.572369 61.205226) (width 0.25) (layer B.Cu) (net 2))
 (segment (start 125.023907 58.408332) (end 126.441577 58.408332) (width 0.25) (layer B.Cu) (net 2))
 (segment (start 126.441577 58.408332) (end 126.638135 58.35333) (width 0.25) (layer B.Cu) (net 2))
 (segment (start 121.138393 59.75238) (end 122.106427 58.784346) (width 0.25) (layer B.Cu) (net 5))
 (segment (start 120.25699 59.75238) (end 121.138393 59.75238) (width 0.25) (layer B.Cu) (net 5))
 (segment (start 119.990576 59.485966) (end 120.25699 59.75238) (width 0.25) (layer B.Cu) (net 5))
 (segment (start 119.566312 59.485966) (end 119.990576 59.485966) (width 0.25) (layer B.Cu) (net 5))
 (via (at 122.788711 58.784346) (size 0.8) (drill 0.4) (layers F.Cu B.Cu) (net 5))
 (segment (start 122.106427 58.784346) (end 122.788711 58.784346) (width 0.25) (layer B.Cu) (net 5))
 (segment (start 125.998057 55.575) (end 131.125 55.575) (width 0.25) (layer F.Cu) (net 5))
 (segment (start 122.788711 58.784346) (end 125.998057 55.575) (width 0.25) (layer F.Cu) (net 5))
 (via (at 131.125 55.575) (size 0.8) (drill 0.4) (layers F.Cu B.Cu) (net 5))
 (segment (start 131.125 55.575) (end 132.125 54.575) (width 0.25) (layer B.Cu) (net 5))
 (segment (start 132.125 54.575) (end 132.125 52.0161) (width 0.25) (layer B.Cu) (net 5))
 (segment (start 125.8189 47.15) (end 125.8189 48.25) (width 0.25) (layer B.Cu) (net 5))
 (segment (start 125.893901 47.074999) (end 125.8189 47.15) (width 0.25) (layer B.Cu) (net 5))
 (segment (start 128.922901 47.074999) (end 125.893901 47.074999) (width 0.25) (layer B.Cu) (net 5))
 (segment (start 129.723899 47.875997) (end 128.922901 47.074999) (width 0.25) (layer B.Cu) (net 5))
 (segment (start 129.723899 49.614999) (end 129.723899 47.875997) (width 0.25) (layer B.Cu) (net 5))
 (segment (start 132.125 52.0161) (end 129.723899 49.614999) (width 0.25) (layer B.Cu) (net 5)))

